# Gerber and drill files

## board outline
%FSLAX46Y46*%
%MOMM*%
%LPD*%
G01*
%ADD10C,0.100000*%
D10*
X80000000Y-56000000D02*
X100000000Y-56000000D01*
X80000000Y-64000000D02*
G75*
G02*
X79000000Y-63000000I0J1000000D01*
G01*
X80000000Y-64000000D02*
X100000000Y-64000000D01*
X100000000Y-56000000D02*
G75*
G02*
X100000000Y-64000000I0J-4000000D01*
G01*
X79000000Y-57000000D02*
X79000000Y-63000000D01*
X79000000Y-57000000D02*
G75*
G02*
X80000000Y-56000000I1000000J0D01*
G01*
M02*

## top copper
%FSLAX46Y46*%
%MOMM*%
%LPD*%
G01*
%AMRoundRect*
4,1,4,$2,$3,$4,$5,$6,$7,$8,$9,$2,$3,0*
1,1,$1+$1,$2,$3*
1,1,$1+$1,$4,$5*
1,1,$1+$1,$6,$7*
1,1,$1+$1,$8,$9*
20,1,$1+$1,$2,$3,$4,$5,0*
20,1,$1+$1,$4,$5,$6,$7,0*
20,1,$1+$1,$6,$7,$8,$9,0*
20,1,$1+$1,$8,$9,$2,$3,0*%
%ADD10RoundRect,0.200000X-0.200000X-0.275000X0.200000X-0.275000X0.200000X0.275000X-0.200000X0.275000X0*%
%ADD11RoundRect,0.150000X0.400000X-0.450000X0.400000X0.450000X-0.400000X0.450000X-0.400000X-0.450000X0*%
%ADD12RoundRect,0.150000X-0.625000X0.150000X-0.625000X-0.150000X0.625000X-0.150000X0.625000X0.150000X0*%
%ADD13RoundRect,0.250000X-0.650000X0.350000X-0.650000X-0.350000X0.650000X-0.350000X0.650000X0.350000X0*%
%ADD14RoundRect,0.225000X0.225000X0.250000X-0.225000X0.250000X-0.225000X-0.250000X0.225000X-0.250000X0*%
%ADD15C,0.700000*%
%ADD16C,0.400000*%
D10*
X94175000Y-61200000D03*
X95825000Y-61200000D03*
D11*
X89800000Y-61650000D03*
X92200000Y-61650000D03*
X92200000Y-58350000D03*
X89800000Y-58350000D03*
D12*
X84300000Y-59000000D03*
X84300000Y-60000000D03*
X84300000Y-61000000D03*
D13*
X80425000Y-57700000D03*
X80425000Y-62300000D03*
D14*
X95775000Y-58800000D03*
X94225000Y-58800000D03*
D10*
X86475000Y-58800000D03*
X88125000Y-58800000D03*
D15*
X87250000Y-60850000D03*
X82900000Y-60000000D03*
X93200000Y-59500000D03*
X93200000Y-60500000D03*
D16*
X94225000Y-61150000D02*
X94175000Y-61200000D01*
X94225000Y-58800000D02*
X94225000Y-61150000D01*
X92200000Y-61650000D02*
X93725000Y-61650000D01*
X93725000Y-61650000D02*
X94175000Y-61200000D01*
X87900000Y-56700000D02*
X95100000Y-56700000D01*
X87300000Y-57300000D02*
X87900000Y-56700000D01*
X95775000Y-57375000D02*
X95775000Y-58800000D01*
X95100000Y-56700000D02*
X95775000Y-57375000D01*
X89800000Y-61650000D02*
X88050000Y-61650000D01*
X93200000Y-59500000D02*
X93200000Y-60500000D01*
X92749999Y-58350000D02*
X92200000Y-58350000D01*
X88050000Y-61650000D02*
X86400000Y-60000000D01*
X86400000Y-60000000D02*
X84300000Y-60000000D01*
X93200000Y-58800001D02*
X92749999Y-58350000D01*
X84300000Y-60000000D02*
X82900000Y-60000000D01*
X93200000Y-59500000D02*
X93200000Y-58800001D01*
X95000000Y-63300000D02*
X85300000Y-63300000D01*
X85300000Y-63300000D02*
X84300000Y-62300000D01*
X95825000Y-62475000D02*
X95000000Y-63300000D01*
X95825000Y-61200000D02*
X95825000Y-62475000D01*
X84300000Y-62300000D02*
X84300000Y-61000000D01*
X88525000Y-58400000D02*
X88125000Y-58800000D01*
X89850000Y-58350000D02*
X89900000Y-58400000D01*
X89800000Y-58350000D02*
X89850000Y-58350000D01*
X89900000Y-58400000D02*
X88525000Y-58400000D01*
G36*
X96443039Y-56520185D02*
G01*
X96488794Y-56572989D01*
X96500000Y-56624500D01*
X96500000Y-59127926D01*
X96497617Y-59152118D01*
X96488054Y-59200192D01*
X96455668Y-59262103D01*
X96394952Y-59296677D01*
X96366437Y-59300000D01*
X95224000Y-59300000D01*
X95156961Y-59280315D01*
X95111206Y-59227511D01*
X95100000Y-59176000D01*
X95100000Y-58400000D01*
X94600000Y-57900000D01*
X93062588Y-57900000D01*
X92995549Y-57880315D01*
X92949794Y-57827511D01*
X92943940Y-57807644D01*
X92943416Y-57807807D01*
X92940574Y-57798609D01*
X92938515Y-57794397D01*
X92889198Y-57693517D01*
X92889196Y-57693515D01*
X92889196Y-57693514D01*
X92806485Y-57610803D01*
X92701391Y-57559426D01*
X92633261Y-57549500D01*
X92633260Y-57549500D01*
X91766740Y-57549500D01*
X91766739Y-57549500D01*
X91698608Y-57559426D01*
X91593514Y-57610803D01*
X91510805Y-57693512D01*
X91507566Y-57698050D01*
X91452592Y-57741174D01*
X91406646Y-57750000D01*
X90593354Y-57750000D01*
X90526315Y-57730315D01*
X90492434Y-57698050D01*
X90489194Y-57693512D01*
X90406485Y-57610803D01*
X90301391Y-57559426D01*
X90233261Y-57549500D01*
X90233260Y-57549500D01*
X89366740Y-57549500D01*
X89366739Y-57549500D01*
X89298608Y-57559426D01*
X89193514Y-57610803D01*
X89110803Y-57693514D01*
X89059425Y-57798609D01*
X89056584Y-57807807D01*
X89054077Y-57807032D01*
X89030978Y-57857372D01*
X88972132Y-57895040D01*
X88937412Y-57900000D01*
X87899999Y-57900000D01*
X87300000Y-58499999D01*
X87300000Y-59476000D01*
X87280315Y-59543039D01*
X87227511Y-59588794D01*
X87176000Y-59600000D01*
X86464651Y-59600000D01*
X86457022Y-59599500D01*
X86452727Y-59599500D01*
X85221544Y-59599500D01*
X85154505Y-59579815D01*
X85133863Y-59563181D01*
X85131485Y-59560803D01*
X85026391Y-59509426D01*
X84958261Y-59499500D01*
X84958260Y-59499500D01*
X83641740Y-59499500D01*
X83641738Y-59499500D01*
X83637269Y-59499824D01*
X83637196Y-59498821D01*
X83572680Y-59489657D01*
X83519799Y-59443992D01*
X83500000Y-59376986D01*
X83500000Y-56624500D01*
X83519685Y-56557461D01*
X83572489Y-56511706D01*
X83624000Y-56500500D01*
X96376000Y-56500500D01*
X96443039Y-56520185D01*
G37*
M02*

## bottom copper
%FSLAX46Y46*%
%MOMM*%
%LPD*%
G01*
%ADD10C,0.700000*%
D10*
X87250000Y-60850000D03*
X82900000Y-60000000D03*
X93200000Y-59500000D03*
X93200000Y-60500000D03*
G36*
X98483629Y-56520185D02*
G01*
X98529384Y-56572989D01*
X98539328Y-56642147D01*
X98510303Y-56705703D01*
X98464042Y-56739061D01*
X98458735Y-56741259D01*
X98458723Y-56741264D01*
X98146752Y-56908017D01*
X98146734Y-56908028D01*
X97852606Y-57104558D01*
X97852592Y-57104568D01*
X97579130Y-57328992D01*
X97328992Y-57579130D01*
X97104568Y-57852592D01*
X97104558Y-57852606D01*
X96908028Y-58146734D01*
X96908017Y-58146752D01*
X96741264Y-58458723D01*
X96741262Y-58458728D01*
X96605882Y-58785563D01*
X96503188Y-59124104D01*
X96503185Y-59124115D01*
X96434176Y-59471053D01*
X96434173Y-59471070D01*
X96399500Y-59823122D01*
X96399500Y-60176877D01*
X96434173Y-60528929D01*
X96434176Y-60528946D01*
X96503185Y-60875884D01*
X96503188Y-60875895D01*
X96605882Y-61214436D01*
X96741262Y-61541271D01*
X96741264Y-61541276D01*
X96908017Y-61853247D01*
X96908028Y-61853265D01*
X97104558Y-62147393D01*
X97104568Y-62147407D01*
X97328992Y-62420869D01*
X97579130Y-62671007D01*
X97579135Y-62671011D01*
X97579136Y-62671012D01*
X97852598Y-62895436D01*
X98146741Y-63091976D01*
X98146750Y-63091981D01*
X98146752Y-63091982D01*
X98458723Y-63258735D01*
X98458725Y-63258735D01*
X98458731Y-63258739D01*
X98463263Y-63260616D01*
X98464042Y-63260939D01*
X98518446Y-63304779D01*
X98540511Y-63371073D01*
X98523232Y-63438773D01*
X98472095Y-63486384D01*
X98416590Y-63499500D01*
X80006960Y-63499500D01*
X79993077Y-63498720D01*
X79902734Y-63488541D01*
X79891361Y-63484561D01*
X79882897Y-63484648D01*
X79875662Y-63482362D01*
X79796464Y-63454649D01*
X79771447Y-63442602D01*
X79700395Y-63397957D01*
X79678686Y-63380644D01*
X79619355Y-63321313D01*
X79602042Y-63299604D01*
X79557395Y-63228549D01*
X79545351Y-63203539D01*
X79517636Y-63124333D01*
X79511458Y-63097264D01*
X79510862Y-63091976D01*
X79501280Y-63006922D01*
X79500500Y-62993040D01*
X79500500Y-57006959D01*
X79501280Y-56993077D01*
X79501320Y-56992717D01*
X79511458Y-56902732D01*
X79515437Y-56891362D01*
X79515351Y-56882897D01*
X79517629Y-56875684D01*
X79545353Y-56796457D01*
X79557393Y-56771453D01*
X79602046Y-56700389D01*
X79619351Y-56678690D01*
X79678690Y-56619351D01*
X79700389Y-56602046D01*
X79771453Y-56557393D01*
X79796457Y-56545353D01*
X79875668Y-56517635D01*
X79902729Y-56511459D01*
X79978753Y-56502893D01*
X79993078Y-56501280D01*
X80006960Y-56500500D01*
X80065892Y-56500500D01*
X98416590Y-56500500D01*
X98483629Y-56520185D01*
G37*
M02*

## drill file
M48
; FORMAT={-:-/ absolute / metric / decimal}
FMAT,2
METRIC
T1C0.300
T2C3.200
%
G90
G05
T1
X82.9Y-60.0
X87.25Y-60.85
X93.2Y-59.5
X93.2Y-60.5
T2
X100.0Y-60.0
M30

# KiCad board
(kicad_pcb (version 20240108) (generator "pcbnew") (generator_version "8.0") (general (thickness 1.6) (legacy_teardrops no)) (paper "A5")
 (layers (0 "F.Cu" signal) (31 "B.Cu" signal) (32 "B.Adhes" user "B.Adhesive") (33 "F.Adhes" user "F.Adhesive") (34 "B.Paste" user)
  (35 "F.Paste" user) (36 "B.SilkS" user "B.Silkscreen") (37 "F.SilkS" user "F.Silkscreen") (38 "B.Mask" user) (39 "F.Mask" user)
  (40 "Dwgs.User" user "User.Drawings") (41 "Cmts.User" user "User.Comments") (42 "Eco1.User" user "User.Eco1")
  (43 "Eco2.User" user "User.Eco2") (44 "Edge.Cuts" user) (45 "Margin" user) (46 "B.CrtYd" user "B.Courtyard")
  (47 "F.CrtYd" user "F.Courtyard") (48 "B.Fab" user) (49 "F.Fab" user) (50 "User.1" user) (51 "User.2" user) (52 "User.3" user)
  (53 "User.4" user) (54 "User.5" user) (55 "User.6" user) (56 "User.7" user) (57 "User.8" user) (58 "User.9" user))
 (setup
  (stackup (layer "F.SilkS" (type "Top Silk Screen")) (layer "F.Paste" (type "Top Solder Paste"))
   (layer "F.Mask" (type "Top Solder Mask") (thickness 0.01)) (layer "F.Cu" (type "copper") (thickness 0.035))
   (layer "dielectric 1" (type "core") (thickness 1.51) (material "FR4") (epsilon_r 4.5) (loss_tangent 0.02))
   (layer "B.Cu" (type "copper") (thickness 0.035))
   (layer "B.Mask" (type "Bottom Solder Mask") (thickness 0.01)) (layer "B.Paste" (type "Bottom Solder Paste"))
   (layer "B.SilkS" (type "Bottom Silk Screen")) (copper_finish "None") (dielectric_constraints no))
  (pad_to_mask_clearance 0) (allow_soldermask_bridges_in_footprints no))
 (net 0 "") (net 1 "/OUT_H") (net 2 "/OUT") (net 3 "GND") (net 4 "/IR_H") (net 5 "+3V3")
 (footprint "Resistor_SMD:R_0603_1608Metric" (layer "F.Cu") (at 95 61.2)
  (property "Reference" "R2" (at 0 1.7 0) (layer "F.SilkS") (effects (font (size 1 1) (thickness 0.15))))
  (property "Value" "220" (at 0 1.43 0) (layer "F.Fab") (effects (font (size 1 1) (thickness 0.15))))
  (pad "1" smd roundrect (at -0.825 0) (size 0.8 0.95) (layers "F.Cu" "F.Paste" "F.Mask") (roundrect_rratio 0.25) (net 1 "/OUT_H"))
  (pad "2" smd roundrect (at 0.825 0) (size 0.8 0.95) (layers "F.Cu" "F.Paste" "F.Mask") (roundrect_rratio 0.25) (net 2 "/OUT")))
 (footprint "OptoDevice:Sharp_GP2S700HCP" (layer "F.Cu") (at 91 60 90)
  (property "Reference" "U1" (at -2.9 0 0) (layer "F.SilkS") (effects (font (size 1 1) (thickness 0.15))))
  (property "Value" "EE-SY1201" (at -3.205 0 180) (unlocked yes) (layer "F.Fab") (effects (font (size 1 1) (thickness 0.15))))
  (pad "1" smd roundrect (at -1.65 -1.2 90) (size 1.2 1.1) (layers "F.Cu" "F.Paste" "F.Mask") (roundrect_rratio 0.1363636364) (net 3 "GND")
   (thermal_bridge_angle 45))
  (pad "2" smd roundrect (at -1.65 1.2 90) (size 1.2 1.1) (layers "F.Cu" "F.Paste" "F.Mask") (roundrect_rratio 0.1363636364)
   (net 1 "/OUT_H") (thermal_bridge_angle 45))
  (pad "3" smd roundrect (at 1.65 1.2 90) (size 1.2 1.1) (layers "F.Cu" "F.Paste" "F.Mask") (roundrect_rratio 0.1363636364) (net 3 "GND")
   (thermal_bridge_angle 45))
  (pad "4" smd roundrect (at 1.65 -1.2 90) (size 1.2 1.1) (layers "F.Cu" "F.Paste" "F.Mask") (roundrect_rratio 0.1363636364) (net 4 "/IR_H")
   (thermal_bridge_angle 45))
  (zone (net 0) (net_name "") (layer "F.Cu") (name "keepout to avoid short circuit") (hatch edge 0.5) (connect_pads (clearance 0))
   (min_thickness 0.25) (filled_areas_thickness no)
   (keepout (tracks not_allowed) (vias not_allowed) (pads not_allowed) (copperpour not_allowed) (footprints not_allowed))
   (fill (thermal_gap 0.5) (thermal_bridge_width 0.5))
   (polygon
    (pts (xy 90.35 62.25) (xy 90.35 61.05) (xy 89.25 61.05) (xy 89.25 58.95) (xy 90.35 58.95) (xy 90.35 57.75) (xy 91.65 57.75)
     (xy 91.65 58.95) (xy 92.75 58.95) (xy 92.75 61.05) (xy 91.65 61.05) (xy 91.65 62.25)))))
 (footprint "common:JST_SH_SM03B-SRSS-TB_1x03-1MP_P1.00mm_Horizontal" (layer "F.Cu") (at 82.3 60 -90)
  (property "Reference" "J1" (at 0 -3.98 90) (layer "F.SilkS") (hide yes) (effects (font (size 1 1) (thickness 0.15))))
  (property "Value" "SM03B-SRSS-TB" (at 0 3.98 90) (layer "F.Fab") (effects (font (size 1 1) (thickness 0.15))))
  (pad "1" smd roundrect (at -1 -2 270) (size 0.6 1.55) (layers "F.Cu" "F.Paste" "F.Mask") (roundrect_rratio 0.25) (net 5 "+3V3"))
  (pad "2" smd roundrect (at 0 -2 270) (size 0.6 1.55) (layers "F.Cu" "F.Paste" "F.Mask") (roundrect_rratio 0.25) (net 3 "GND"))
  (pad "3" smd roundrect (at 1 -2 270) (size 0.6 1.55) (layers "F.Cu" "F.Paste" "F.Mask") (roundrect_rratio 0.25) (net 2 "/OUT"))
  (pad "MP" smd roundrect (at -2.3 1.875 270) (size 1.2 1.8) (layers "F.Cu" "F.Paste" "F.Mask") (roundrect_rratio 0.208333))
  (pad "MP" smd roundrect (at 2.3 1.875 270) (size 1.2 1.8) (layers "F.Cu" "F.Paste" "F.Mask") (roundrect_rratio 0.208333)))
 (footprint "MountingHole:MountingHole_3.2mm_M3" (layer "F.Cu") (at 100 60)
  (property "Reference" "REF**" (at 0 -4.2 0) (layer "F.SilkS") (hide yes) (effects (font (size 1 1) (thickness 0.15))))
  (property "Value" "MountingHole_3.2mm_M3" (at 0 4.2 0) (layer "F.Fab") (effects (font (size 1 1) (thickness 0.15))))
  (pad "" np_thru_hole circle (at 0 0) (size 3.2 3.2) (drill 3.2) (layers "F&B.Cu" "*.Mask") (solder_mask_margin 1.9) (clearance 2)))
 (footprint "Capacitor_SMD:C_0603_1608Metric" (layer "F.Cu") (at 95 58.8 180)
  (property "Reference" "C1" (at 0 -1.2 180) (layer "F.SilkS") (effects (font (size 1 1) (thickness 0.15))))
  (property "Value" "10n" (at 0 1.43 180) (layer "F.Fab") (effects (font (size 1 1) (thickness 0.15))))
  (pad "1" smd roundrect (at -0.775 0 180) (size 0.9 0.95) (layers "F.Cu" "F.Paste" "F.Mask") (roundrect_rratio 0.25) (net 5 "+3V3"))
  (pad "2" smd roundrect (at 0.775 0 180) (size 0.9 0.95) (layers "F.Cu" "F.Paste" "F.Mask") (roundrect_rratio 0.25) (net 1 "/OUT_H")))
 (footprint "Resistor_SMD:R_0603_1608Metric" (layer "F.Cu") (at 87.3 58.8)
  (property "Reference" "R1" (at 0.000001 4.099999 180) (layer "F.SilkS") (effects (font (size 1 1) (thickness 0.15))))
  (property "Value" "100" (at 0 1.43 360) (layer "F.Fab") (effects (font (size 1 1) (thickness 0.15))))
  (pad "1" smd roundrect (at -0.825 0) (size 0.8 0.95) (layers "F.Cu" "F.Paste" "F.Mask") (roundrect_rratio 0.25) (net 5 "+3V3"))
  (pad "2" smd roundrect (at 0.825 0) (size 0.8 0.95) (layers "F.Cu" "F.Paste" "F.Mask") (roundrect_rratio 0.25) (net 4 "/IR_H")))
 (gr_line (start 80 56) (end 100 56) (stroke (width 0.1) (type default)) (layer "Edge.Cuts"))
 (gr_arc (start 80 64) (mid 79.292893 63.707107) (end 79 63) (stroke (width 0.1) (type default)) (layer "Edge.Cuts"))
 (gr_line (start 80 64) (end 100 64) (stroke (width 0.1) (type default)) (layer "Edge.Cuts"))
 (gr_arc (start 100 56) (mid 104 60) (end 100 64) (stroke (width 0.1) (type default)) (layer "Edge.Cuts"))
 (gr_line (start 79 57) (end 79 63) (stroke (width 0.1) (type default)) (layer "Edge.Cuts"))
 (gr_arc (start 79 57) (mid 79.292893 56.292893) (end 80 56) (stroke (width 0.1) (type default)) (layer "Edge.Cuts"))
 (segment (start 94.225 61.15) (end 94.175 61.2) (width 0.4) (layer "F.Cu") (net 1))
 (segment (start 94.225 58.8) (end 94.225 61.15) (width 0.4) (layer "F.Cu") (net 1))
 (segment (start 92.2 61.65) (end 93.725 61.65) (width 0.4) (layer "F.Cu") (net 1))
 (segment (start 93.725 61.65) (end 94.175 61.2) (width 0.4) (layer "F.Cu") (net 1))
 (segment (start 87.9 56.7) (end 95.1 56.7) (width 0.4) (layer "F.Cu") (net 5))
 (segment (start 87.3 57.3) (end 87.9 56.7) (width 0.4) (layer "F.Cu") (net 5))
 (segment (start 95.775 57.375) (end 95.775 58.8) (width 0.4) (layer "F.Cu") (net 5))
 (segment (start 95.1 56.7) (end 95.775 57.375) (width 0.4) (layer "F.Cu") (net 5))
 (segment (start 89.8 61.65) (end 88.05 61.65) (width 0.4) (layer "F.Cu") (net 3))
 (segment (start 93.2 59.5) (end 93.2 60.5) (width 0.4) (layer "F.Cu") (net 3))
 (segment (start 92.749999 58.35) (end 92.2 58.35) (width 0.4) (layer "F.Cu") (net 3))
 (segment (start 88.05 61.65) (end 86.4 60) (width 0.4) (layer "F.Cu") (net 3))
 (segment (start 86.4 60) (end 84.3 60) (width 0.4) (layer "F.Cu") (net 3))
 (segment (start 93.2 58.800001) (end 92.749999 58.35) (width 0.4) (layer "F.Cu") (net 3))
 (segment (start 84.3 60) (end 82.9 60) (width 0.4) (layer "F.Cu") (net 3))
 (segment (start 93.2 59.5) (end 93.2 58.800001) (width 0.4) (layer "F.Cu") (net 3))
 (via (at 87.25 60.85) (size 0.7) (drill 0.3) (layers "F.Cu" "B.Cu") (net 3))
 (via (at 82.9 60) (size 0.7) (drill 0.3) (layers "F.Cu" "B.Cu") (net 3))
 (via (at 93.2 59.5) (size 0.7) (drill 0.3) (layers "F.Cu" "B.Cu") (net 3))
 (via (at 93.2 60.5) (size 0.7) (drill 0.3) (layers "F.Cu" "B.Cu") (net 3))
 (segment (start 95 63.3) (end 85.3 63.3) (width 0.4) (layer "F.Cu") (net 2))
 (segment (start 85.3 63.3) (end 84.3 62.3) (width 0.4) (layer "F.Cu") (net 2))
 (segment (start 95.825 62.475) (end 95 63.3) (width 0.4) (layer "F.Cu") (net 2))
 (segment (start 95.825 61.2) (end 95.825 62.475) (width 0.4) (layer "F.Cu") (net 2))
 (segment (start 84.3 62.3) (end 84.3 61) (width 0.4) (layer "F.Cu") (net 2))
 (segment (start 88.525 58.4) (end 88.125 58.8) (width 0.4) (layer "F.Cu") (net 4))
 (segment (start 89.85 58.35) (end 89.9 58.4) (width 0.4) (layer "F.Cu") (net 4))
 (segment (start 89.8 58.35) (end 89.85 58.35) (width 0.4) (layer "F.Cu") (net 4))
 (segment (start 89.9 58.4) (end 88.525 58.4) (width 0.4) (layer "F.Cu") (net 4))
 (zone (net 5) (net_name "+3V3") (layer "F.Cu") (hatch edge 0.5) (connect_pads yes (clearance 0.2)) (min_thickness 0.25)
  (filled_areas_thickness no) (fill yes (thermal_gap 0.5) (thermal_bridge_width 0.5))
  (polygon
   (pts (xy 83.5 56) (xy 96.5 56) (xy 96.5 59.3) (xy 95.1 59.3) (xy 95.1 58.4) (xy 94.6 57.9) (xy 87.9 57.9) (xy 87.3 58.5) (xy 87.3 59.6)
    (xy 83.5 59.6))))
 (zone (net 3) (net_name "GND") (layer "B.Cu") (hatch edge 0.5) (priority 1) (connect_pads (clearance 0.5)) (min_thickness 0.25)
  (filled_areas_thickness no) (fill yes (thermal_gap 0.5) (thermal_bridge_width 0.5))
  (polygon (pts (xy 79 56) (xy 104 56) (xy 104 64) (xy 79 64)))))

